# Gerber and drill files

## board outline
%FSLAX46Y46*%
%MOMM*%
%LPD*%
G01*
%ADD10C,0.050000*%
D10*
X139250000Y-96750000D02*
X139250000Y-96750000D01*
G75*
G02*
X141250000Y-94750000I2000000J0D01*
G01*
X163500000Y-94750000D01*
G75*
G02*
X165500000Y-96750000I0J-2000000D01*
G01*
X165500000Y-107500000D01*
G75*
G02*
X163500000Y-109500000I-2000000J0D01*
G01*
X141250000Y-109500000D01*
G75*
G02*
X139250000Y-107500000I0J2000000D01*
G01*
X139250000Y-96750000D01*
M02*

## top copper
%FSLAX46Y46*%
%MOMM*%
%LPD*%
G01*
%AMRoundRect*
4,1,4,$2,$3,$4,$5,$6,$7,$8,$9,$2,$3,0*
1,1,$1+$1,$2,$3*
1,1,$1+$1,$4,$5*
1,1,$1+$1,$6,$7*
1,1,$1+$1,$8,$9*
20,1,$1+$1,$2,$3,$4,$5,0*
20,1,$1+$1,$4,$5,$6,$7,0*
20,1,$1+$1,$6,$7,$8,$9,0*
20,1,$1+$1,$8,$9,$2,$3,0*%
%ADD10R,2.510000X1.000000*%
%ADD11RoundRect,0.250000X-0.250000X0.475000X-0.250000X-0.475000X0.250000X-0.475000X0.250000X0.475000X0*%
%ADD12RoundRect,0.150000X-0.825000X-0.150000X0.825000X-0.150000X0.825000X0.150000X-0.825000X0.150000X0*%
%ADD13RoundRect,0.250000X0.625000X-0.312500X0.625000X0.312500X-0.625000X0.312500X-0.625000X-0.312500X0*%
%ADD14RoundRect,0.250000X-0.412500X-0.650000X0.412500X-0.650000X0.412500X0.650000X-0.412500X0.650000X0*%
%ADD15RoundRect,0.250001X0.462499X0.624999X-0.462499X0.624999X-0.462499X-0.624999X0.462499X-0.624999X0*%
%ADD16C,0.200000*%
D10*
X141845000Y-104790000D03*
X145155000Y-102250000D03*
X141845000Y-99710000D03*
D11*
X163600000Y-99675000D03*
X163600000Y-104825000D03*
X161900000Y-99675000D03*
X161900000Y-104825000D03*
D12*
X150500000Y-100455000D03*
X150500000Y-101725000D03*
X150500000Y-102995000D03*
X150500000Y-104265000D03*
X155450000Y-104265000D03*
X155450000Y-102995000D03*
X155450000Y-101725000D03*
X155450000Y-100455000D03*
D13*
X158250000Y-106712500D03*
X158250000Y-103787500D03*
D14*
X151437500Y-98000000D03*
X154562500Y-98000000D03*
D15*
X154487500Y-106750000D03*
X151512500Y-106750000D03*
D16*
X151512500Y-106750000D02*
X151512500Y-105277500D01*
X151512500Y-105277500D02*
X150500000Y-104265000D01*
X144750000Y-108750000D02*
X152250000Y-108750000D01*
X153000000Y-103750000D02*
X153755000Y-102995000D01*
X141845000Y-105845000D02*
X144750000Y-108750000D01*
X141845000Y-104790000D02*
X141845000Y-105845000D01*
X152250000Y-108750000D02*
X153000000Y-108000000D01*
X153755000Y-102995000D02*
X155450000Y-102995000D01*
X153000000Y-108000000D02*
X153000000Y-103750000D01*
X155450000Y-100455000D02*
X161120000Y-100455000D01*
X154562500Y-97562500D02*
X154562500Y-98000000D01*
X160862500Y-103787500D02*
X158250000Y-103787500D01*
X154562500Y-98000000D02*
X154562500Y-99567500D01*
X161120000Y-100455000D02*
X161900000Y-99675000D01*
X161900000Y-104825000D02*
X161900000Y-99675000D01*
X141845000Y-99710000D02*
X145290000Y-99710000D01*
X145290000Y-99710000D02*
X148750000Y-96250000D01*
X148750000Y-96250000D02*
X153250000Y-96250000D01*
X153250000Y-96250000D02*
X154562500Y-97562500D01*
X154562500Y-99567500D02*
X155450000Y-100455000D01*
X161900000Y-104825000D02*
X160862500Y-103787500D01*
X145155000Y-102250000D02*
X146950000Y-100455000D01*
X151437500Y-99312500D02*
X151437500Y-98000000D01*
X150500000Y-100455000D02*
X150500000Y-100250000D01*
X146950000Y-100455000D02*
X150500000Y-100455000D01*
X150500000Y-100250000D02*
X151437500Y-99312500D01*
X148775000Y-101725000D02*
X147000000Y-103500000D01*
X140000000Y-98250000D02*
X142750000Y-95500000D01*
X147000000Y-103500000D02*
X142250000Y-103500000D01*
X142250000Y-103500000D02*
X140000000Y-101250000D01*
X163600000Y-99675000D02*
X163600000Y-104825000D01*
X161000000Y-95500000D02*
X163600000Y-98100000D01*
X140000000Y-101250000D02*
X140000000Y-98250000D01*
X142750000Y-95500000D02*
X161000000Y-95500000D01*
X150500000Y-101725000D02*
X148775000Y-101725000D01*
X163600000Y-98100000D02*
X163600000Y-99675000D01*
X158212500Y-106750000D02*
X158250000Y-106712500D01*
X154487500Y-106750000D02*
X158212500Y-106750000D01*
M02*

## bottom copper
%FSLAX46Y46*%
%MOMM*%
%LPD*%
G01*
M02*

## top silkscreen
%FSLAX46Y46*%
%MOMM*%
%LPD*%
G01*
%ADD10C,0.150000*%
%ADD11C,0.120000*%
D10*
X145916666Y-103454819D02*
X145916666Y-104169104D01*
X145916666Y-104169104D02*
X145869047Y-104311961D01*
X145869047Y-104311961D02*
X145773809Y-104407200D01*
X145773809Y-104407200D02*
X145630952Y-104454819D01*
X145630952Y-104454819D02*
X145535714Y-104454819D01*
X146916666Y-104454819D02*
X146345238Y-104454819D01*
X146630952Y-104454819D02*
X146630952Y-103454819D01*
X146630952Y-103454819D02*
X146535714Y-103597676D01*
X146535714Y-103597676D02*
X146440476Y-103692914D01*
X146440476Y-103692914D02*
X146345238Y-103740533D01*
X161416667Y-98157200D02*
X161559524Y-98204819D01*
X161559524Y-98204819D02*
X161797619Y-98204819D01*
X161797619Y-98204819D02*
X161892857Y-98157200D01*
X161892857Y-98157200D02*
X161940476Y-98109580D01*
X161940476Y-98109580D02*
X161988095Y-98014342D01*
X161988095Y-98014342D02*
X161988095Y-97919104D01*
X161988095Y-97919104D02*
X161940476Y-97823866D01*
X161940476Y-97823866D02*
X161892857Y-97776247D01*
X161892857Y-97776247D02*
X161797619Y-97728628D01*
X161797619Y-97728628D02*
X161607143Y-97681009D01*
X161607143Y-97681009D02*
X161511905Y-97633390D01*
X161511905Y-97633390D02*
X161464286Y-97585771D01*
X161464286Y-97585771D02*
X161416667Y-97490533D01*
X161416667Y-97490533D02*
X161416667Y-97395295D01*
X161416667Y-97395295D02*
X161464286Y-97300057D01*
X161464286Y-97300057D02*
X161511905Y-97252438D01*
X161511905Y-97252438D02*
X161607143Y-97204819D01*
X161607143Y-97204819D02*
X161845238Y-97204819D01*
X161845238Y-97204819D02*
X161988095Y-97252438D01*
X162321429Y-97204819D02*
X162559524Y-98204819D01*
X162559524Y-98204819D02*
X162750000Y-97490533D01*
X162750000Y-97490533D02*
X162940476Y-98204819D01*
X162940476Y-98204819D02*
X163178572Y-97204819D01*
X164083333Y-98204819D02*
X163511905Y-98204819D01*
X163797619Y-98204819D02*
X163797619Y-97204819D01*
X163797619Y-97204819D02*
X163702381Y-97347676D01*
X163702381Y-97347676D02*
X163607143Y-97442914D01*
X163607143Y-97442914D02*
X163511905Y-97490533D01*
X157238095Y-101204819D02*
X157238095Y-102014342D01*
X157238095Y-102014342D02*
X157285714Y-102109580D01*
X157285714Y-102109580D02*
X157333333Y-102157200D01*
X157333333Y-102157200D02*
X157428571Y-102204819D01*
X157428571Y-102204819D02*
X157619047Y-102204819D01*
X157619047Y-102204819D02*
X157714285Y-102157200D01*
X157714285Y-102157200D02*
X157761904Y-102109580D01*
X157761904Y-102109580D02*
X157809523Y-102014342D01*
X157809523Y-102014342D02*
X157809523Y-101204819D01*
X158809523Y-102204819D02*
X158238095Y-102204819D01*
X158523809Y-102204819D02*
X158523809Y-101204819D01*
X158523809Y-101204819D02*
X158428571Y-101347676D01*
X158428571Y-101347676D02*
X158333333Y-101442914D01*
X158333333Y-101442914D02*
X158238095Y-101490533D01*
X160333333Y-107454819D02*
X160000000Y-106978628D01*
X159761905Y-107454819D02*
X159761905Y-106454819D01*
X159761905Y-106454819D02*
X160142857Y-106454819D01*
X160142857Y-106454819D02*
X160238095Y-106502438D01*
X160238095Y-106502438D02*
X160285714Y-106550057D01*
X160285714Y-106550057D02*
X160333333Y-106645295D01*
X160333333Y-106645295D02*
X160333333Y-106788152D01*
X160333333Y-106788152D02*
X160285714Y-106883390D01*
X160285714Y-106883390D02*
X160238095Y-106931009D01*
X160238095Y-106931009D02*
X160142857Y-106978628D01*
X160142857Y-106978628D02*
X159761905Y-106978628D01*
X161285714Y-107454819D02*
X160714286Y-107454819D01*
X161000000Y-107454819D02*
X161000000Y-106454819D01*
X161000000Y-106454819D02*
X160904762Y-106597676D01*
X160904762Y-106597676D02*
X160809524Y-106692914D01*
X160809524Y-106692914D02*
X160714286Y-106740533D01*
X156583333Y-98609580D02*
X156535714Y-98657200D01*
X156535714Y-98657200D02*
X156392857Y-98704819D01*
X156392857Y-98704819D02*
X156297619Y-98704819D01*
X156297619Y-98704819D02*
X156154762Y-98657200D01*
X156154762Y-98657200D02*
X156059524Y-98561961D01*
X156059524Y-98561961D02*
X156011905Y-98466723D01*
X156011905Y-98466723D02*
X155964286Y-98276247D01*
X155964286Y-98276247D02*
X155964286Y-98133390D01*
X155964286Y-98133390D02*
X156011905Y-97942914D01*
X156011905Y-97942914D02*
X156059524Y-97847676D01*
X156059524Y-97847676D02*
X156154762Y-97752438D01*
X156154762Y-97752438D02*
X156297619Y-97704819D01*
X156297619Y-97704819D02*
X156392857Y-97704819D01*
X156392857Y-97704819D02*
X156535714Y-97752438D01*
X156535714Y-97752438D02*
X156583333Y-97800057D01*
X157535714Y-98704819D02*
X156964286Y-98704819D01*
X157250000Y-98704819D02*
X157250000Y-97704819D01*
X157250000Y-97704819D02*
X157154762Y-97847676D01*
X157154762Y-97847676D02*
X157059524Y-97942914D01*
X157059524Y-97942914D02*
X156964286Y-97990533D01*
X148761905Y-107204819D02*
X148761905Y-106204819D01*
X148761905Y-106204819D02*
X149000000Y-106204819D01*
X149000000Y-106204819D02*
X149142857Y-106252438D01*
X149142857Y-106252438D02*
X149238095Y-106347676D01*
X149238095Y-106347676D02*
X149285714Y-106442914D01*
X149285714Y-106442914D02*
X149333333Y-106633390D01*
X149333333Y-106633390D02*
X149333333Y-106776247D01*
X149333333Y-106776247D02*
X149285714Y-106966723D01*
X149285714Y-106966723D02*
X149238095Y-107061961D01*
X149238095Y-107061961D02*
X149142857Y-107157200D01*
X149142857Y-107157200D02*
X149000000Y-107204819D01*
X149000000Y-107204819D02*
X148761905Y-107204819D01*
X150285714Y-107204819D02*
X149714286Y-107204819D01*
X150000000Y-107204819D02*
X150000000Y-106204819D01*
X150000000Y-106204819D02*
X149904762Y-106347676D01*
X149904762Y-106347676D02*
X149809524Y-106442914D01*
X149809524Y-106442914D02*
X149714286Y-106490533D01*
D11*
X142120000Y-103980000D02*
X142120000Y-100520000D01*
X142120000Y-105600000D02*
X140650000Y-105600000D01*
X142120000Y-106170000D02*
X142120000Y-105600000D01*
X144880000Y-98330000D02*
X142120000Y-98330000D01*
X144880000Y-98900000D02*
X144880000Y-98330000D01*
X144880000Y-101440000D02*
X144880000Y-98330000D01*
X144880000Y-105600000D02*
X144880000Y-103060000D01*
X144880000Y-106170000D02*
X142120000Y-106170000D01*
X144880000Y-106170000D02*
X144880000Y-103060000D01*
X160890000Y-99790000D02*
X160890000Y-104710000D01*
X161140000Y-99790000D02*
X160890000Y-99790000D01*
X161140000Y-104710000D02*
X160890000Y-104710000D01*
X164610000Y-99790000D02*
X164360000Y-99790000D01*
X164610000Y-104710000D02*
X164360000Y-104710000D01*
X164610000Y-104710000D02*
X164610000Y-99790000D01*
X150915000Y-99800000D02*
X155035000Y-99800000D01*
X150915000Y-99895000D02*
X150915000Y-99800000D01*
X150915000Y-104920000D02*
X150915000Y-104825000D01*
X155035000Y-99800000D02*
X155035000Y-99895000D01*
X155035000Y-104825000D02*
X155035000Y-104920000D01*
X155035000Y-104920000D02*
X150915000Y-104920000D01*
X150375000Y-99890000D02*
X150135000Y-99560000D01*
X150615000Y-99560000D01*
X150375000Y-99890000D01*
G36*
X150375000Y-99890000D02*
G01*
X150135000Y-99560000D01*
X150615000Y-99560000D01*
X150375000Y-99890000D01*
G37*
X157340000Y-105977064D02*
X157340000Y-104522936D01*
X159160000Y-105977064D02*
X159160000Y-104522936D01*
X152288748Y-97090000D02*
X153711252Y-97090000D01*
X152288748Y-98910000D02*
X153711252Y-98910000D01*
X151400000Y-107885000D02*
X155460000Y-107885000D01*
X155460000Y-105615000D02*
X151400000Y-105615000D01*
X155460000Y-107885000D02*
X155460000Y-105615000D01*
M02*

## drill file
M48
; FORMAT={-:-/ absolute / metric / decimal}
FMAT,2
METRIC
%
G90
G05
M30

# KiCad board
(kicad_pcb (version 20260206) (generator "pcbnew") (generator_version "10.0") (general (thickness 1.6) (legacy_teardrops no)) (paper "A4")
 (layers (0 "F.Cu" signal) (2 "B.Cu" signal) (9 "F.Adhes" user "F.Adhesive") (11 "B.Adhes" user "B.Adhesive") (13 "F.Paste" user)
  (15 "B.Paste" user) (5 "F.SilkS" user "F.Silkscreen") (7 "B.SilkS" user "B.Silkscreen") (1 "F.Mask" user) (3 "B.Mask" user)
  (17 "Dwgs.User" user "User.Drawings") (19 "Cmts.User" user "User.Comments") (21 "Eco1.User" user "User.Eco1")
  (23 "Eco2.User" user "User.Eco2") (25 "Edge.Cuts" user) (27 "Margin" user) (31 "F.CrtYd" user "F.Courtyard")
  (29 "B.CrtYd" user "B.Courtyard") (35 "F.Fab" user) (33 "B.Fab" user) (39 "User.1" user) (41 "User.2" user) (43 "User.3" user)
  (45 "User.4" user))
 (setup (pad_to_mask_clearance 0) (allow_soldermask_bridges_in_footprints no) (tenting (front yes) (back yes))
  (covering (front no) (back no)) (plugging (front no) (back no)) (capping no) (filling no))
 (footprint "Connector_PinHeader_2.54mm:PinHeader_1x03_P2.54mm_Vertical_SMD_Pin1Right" (layer "F.Cu") (at 143.5 102.25 180)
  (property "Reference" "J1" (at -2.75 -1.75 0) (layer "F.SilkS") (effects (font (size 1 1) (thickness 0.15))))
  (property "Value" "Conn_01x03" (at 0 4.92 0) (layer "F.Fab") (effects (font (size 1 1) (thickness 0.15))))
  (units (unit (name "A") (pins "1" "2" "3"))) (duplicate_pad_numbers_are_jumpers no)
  (fp_line (start 1.38 -1.73) (end 1.38 1.73) (stroke (width 0.12) (type solid)) (layer "F.SilkS"))
  (fp_line (start 1.38 -3.35) (end 2.85 -3.35) (stroke (width 0.12) (type solid)) (layer "F.SilkS"))
  (fp_line (start 1.38 -3.92) (end 1.38 -3.35) (stroke (width 0.12) (type solid)) (layer "F.SilkS"))
  (fp_line (start -1.38 3.92) (end 1.38 3.92) (stroke (width 0.12) (type solid)) (layer "F.SilkS"))
  (fp_line (start -1.38 3.35) (end -1.38 3.92) (stroke (width 0.12) (type solid)) (layer "F.SilkS"))
  (fp_line (start -1.38 0.81) (end -1.38 3.92) (stroke (width 0.12) (type solid)) (layer "F.SilkS"))
  (fp_line (start -1.38 -3.35) (end -1.38 -0.81) (stroke (width 0.12) (type solid)) (layer "F.SilkS"))
  (fp_line (start -1.38 -3.92) (end 1.38 -3.92) (stroke (width 0.12) (type solid)) (layer "F.SilkS"))
  (fp_line (start -1.38 -3.92) (end -1.38 -0.81) (stroke (width 0.12) (type solid)) (layer "F.SilkS"))
  (pad "1" smd rect (at 1.655 -2.54 180) (size 2.51 1) (layers "F.Cu" "F.Mask" "F.Paste") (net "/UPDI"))
  (pad "2" smd rect (at -1.655 0 180) (size 2.51 1) (layers "F.Cu" "F.Mask" "F.Paste") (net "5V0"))
  (pad "3" smd rect (at 1.655 2.54 180) (size 2.51 1) (layers "F.Cu" "F.Mask" "F.Paste") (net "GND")))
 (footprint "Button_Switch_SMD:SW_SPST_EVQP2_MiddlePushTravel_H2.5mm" (layer "F.Cu") (at 162.75 102.25 -90)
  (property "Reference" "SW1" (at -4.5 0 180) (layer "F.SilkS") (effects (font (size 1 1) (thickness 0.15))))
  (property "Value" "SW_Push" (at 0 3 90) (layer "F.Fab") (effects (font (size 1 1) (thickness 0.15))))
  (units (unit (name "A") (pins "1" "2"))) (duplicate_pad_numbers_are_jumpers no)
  (fp_line (start -2.46 1.86) (end 2.46 1.86) (stroke (width 0.12) (type solid)) (layer "F.SilkS"))
  (fp_line (start -2.46 1.61) (end -2.46 1.86) (stroke (width 0.12) (type solid)) (layer "F.SilkS"))
  (fp_line (start 2.46 1.61) (end 2.46 1.86) (stroke (width 0.12) (type solid)) (layer "F.SilkS"))
  (fp_line (start -2.46 -1.86) (end -2.46 -1.61) (stroke (width 0.12) (type solid)) (layer "F.SilkS"))
  (fp_line (start 2.46 -1.86) (end 2.46 -1.61) (stroke (width 0.12) (type solid)) (layer "F.SilkS"))
  (fp_line (start 2.46 -1.86) (end -2.46 -1.86) (stroke (width 0.12) (type solid)) (layer "F.SilkS"))
  (pad "1" smd roundrect (at -2.575 -0.85 270) (size 1.45 1) (layers "F.Cu" "F.Mask" "F.Paste") (roundrect_rratio 0.25) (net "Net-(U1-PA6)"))
  (pad "1" smd roundrect (at 2.575 -0.85 270) (size 1.45 1) (layers "F.Cu" "F.Mask" "F.Paste") (roundrect_rratio 0.25) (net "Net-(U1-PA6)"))
  (pad "2" smd roundrect (at -2.575 0.85 270) (size 1.45 1) (layers "F.Cu" "F.Mask" "F.Paste") (roundrect_rratio 0.25) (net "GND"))
  (pad "2" smd roundrect (at 2.575 0.85 270) (size 1.45 1) (layers "F.Cu" "F.Mask" "F.Paste") (roundrect_rratio 0.25) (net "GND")))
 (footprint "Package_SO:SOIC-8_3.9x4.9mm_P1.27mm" (layer "F.Cu") (at 152.975 102.36)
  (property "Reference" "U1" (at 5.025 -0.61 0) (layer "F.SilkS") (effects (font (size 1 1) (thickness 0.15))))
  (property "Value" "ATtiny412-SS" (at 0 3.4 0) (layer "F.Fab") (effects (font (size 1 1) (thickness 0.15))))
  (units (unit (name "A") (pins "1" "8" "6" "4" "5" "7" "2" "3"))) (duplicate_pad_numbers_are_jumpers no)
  (fp_line (start -2.06 -2.56) (end 2.06 -2.56) (stroke (width 0.12) (type solid)) (layer "F.SilkS"))
  (fp_line (start -2.06 -2.465) (end -2.06 -2.56) (stroke (width 0.12) (type solid)) (layer "F.SilkS"))
  (fp_line (start -2.06 2.56) (end -2.06 2.465) (stroke (width 0.12) (type solid)) (layer "F.SilkS"))
  (fp_line (start 2.06 -2.56) (end 2.06 -2.465) (stroke (width 0.12) (type solid)) (layer "F.SilkS"))
  (fp_line (start 2.06 2.465) (end 2.06 2.56) (stroke (width 0.12) (type solid)) (layer "F.SilkS"))
  (fp_line (start 2.06 2.56) (end -2.06 2.56) (stroke (width 0.12) (type solid)) (layer "F.SilkS"))
  (fp_poly (pts (xy -2.6 -2.47) (xy -2.84 -2.8) (xy -2.36 -2.8)) (stroke (width 0.12) (type solid)) (fill yes) (layer "F.SilkS"))
  (pad "1" smd roundrect (at -2.475 -1.905) (size 1.95 0.6) (layers "F.Cu" "F.Mask" "F.Paste") (roundrect_rratio 0.25) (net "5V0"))
  (pad "2" smd roundrect (at -2.475 -0.635) (size 1.95 0.6) (layers "F.Cu" "F.Mask" "F.Paste") (roundrect_rratio 0.25) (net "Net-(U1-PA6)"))
  (pad "3" smd roundrect (at -2.475 0.635) (size 1.95 0.6) (layers "F.Cu" "F.Mask" "F.Paste") (roundrect_rratio 0.25)
   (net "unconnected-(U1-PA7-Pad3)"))
  (pad "4" smd roundrect (at -2.475 1.905) (size 1.95 0.6) (layers "F.Cu" "F.Mask" "F.Paste") (roundrect_rratio 0.25) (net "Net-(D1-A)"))
  (pad "5" smd roundrect (at 2.475 1.905) (size 1.95 0.6) (layers "F.Cu" "F.Mask" "F.Paste") (roundrect_rratio 0.25)
   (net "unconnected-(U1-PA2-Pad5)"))
  (pad "6" smd roundrect (at 2.475 0.635) (size 1.95 0.6) (layers "F.Cu" "F.Mask" "F.Paste") (roundrect_rratio 0.25) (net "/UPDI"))
  (pad "7" smd roundrect (at 2.475 -0.635) (size 1.95 0.6) (layers "F.Cu" "F.Mask" "F.Paste") (roundrect_rratio 0.25)
   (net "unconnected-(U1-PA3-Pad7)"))
  (pad "8" smd roundrect (at 2.475 -1.905) (size 1.95 0.6) (layers "F.Cu" "F.Mask" "F.Paste") (roundrect_rratio 0.25) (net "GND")))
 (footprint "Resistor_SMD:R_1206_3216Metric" (layer "F.Cu") (at 158.25 105.25 90)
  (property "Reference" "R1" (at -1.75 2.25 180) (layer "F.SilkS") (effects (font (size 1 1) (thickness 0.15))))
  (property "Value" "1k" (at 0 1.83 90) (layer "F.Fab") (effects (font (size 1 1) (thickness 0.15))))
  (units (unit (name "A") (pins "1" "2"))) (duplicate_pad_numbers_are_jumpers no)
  (fp_line (start -0.727064 -0.91) (end 0.727064 -0.91) (stroke (width 0.12) (type solid)) (layer "F.SilkS"))
  (fp_line (start -0.727064 0.91) (end 0.727064 0.91) (stroke (width 0.12) (type solid)) (layer "F.SilkS"))
  (pad "1" smd roundrect (at -1.4625 0 90) (size 1.125 1.75) (layers "F.Cu" "F.Mask" "F.Paste") (roundrect_rratio 0.222222)
   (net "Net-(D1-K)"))
  (pad "2" smd roundrect (at 1.4625 0 90) (size 1.125 1.75) (layers "F.Cu" "F.Mask" "F.Paste") (roundrect_rratio 0.222222) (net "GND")))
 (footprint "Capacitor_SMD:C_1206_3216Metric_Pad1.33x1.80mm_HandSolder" (layer "F.Cu") (at 153 98)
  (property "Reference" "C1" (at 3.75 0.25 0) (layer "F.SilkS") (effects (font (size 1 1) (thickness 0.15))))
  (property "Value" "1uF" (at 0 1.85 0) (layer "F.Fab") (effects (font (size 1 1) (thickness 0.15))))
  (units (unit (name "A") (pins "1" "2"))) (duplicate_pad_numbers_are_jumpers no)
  (fp_line (start -0.711252 -0.91) (end 0.711252 -0.91) (stroke (width 0.12) (type solid)) (layer "F.SilkS"))
  (fp_line (start -0.711252 0.91) (end 0.711252 0.91) (stroke (width 0.12) (type solid)) (layer "F.SilkS"))
  (pad "1" smd roundrect (at -1.5625 0) (size 1.325 1.8) (layers "F.Cu" "F.Mask" "F.Paste") (roundrect_rratio 0.188679) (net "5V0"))
  (pad "2" smd roundrect (at 1.5625 0) (size 1.325 1.8) (layers "F.Cu" "F.Mask" "F.Paste") (roundrect_rratio 0.188679) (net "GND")))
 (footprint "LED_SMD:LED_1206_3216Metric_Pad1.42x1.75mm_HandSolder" (layer "F.Cu") (at 153 106.75 180)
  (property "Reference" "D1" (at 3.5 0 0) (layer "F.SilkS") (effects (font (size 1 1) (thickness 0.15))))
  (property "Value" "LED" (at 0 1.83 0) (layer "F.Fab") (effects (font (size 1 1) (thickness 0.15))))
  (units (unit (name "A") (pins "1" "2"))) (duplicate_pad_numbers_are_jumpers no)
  (fp_line (start 1.6 -1.135) (end -2.46 -1.135) (stroke (width 0.12) (type solid)) (layer "F.SilkS"))
  (fp_line (start -2.46 1.135) (end 1.6 1.135) (stroke (width 0.12) (type solid)) (layer "F.SilkS"))
  (fp_line (start -2.46 -1.135) (end -2.46 1.135) (stroke (width 0.12) (type solid)) (layer "F.SilkS"))
  (pad "1" smd roundrect (at -1.4875 0 180) (size 1.425 1.75) (layers "F.Cu" "F.Mask" "F.Paste") (roundrect_rratio 0.175439)
   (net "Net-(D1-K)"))
  (pad "2" smd roundrect (at 1.4875 0 180) (size 1.425 1.75) (layers "F.Cu" "F.Mask" "F.Paste") (roundrect_rratio 0.175439)
   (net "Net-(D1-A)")))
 (gr_rect (start 139.25 94.75) (end 165.5 109.5) (radius 2) (stroke (width 0.05) (type solid)) (fill no) (layer "Edge.Cuts"))
 (segment (start 151.5125 106.75) (end 151.5125 105.2775) (width 0.2) (layer "F.Cu") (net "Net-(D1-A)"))
 (segment (start 151.5125 105.2775) (end 150.5 104.265) (width 0.2) (layer "F.Cu") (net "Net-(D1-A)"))
 (segment (start 144.75 108.75) (end 152.25 108.75) (width 0.2) (layer "F.Cu") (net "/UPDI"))
 (segment (start 153 103.75) (end 153.755 102.995) (width 0.2) (layer "F.Cu") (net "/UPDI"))
 (segment (start 141.845 105.845) (end 144.75 108.75) (width 0.2) (layer "F.Cu") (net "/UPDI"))
 (segment (start 141.845 104.79) (end 141.845 105.845) (width 0.2) (layer "F.Cu") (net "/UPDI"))
 (segment (start 152.25 108.75) (end 153 108) (width 0.2) (layer "F.Cu") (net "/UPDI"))
 (segment (start 153.755 102.995) (end 155.45 102.995) (width 0.2) (layer "F.Cu") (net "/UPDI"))
 (segment (start 153 108) (end 153 103.75) (width 0.2) (layer "F.Cu") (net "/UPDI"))
 (segment (start 155.45 100.455) (end 161.12 100.455) (width 0.2) (layer "F.Cu") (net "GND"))
 (segment (start 154.5625 97.5625) (end 154.5625 98) (width 0.2) (layer "F.Cu") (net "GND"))
 (segment (start 160.8625 103.7875) (end 158.25 103.7875) (width 0.2) (layer "F.Cu") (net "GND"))
 (segment (start 154.5625 98) (end 154.5625 99.5675) (width 0.2) (layer "F.Cu") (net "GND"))
 (segment (start 161.12 100.455) (end 161.9 99.675) (width 0.2) (layer "F.Cu") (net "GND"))
 (segment (start 161.9 104.825) (end 161.9 99.675) (width 0.2) (layer "F.Cu") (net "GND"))
 (segment (start 141.845 99.71) (end 145.29 99.71) (width 0.2) (layer "F.Cu") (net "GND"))
 (segment (start 145.29 99.71) (end 148.75 96.25) (width 0.2) (layer "F.Cu") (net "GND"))
 (segment (start 148.75 96.25) (end 153.25 96.25) (width 0.2) (layer "F.Cu") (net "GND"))
 (segment (start 153.25 96.25) (end 154.5625 97.5625) (width 0.2) (layer "F.Cu") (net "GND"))
 (segment (start 154.5625 99.5675) (end 155.45 100.455) (width 0.2) (layer "F.Cu") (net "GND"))
 (segment (start 161.9 104.825) (end 160.8625 103.7875) (width 0.2) (layer "F.Cu") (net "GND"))
 (segment (start 145.155 102.25) (end 146.95 100.455) (width 0.2) (layer "F.Cu") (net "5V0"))
 (segment (start 151.4375 99.3125) (end 151.4375 98) (width 0.2) (layer "F.Cu") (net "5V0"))
 (segment (start 150.5 100.455) (end 150.5 100.25) (width 0.2) (layer "F.Cu") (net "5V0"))
 (segment (start 146.95 100.455) (end 150.5 100.455) (width 0.2) (layer "F.Cu") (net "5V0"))
 (segment (start 150.5 100.25) (end 151.4375 99.3125) (width 0.2) (layer "F.Cu") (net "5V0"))
 (segment (start 148.775 101.725) (end 147 103.5) (width 0.2) (layer "F.Cu") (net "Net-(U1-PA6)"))
 (segment (start 140 98.25) (end 142.75 95.5) (width 0.2) (layer "F.Cu") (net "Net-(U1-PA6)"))
 (segment (start 147 103.5) (end 142.25 103.5) (width 0.2) (layer "F.Cu") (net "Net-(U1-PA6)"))
 (segment (start 142.25 103.5) (end 140 101.25) (width 0.2) (layer "F.Cu") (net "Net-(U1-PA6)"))
 (segment (start 163.6 99.675) (end 163.6 104.825) (width 0.2) (layer "F.Cu") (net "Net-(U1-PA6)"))
 (segment (start 161 95.5) (end 163.6 98.1) (width 0.2) (layer "F.Cu") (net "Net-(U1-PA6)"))
 (segment (start 140 101.25) (end 140 98.25) (width 0.2) (layer "F.Cu") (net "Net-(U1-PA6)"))
 (segment (start 142.75 95.5) (end 161 95.5) (width 0.2) (layer "F.Cu") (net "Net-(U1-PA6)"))
 (segment (start 150.5 101.725) (end 148.775 101.725) (width 0.2) (layer "F.Cu") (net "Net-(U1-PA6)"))
 (segment (start 163.6 98.1) (end 163.6 99.675) (width 0.2) (layer "F.Cu") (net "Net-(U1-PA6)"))
 (segment (start 158.2125 106.75) (end 158.25 106.7125) (width 0.2) (layer "F.Cu") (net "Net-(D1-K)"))
 (segment (start 154.4875 106.75) (end 158.2125 106.75) (width 0.2) (layer "F.Cu") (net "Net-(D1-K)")))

